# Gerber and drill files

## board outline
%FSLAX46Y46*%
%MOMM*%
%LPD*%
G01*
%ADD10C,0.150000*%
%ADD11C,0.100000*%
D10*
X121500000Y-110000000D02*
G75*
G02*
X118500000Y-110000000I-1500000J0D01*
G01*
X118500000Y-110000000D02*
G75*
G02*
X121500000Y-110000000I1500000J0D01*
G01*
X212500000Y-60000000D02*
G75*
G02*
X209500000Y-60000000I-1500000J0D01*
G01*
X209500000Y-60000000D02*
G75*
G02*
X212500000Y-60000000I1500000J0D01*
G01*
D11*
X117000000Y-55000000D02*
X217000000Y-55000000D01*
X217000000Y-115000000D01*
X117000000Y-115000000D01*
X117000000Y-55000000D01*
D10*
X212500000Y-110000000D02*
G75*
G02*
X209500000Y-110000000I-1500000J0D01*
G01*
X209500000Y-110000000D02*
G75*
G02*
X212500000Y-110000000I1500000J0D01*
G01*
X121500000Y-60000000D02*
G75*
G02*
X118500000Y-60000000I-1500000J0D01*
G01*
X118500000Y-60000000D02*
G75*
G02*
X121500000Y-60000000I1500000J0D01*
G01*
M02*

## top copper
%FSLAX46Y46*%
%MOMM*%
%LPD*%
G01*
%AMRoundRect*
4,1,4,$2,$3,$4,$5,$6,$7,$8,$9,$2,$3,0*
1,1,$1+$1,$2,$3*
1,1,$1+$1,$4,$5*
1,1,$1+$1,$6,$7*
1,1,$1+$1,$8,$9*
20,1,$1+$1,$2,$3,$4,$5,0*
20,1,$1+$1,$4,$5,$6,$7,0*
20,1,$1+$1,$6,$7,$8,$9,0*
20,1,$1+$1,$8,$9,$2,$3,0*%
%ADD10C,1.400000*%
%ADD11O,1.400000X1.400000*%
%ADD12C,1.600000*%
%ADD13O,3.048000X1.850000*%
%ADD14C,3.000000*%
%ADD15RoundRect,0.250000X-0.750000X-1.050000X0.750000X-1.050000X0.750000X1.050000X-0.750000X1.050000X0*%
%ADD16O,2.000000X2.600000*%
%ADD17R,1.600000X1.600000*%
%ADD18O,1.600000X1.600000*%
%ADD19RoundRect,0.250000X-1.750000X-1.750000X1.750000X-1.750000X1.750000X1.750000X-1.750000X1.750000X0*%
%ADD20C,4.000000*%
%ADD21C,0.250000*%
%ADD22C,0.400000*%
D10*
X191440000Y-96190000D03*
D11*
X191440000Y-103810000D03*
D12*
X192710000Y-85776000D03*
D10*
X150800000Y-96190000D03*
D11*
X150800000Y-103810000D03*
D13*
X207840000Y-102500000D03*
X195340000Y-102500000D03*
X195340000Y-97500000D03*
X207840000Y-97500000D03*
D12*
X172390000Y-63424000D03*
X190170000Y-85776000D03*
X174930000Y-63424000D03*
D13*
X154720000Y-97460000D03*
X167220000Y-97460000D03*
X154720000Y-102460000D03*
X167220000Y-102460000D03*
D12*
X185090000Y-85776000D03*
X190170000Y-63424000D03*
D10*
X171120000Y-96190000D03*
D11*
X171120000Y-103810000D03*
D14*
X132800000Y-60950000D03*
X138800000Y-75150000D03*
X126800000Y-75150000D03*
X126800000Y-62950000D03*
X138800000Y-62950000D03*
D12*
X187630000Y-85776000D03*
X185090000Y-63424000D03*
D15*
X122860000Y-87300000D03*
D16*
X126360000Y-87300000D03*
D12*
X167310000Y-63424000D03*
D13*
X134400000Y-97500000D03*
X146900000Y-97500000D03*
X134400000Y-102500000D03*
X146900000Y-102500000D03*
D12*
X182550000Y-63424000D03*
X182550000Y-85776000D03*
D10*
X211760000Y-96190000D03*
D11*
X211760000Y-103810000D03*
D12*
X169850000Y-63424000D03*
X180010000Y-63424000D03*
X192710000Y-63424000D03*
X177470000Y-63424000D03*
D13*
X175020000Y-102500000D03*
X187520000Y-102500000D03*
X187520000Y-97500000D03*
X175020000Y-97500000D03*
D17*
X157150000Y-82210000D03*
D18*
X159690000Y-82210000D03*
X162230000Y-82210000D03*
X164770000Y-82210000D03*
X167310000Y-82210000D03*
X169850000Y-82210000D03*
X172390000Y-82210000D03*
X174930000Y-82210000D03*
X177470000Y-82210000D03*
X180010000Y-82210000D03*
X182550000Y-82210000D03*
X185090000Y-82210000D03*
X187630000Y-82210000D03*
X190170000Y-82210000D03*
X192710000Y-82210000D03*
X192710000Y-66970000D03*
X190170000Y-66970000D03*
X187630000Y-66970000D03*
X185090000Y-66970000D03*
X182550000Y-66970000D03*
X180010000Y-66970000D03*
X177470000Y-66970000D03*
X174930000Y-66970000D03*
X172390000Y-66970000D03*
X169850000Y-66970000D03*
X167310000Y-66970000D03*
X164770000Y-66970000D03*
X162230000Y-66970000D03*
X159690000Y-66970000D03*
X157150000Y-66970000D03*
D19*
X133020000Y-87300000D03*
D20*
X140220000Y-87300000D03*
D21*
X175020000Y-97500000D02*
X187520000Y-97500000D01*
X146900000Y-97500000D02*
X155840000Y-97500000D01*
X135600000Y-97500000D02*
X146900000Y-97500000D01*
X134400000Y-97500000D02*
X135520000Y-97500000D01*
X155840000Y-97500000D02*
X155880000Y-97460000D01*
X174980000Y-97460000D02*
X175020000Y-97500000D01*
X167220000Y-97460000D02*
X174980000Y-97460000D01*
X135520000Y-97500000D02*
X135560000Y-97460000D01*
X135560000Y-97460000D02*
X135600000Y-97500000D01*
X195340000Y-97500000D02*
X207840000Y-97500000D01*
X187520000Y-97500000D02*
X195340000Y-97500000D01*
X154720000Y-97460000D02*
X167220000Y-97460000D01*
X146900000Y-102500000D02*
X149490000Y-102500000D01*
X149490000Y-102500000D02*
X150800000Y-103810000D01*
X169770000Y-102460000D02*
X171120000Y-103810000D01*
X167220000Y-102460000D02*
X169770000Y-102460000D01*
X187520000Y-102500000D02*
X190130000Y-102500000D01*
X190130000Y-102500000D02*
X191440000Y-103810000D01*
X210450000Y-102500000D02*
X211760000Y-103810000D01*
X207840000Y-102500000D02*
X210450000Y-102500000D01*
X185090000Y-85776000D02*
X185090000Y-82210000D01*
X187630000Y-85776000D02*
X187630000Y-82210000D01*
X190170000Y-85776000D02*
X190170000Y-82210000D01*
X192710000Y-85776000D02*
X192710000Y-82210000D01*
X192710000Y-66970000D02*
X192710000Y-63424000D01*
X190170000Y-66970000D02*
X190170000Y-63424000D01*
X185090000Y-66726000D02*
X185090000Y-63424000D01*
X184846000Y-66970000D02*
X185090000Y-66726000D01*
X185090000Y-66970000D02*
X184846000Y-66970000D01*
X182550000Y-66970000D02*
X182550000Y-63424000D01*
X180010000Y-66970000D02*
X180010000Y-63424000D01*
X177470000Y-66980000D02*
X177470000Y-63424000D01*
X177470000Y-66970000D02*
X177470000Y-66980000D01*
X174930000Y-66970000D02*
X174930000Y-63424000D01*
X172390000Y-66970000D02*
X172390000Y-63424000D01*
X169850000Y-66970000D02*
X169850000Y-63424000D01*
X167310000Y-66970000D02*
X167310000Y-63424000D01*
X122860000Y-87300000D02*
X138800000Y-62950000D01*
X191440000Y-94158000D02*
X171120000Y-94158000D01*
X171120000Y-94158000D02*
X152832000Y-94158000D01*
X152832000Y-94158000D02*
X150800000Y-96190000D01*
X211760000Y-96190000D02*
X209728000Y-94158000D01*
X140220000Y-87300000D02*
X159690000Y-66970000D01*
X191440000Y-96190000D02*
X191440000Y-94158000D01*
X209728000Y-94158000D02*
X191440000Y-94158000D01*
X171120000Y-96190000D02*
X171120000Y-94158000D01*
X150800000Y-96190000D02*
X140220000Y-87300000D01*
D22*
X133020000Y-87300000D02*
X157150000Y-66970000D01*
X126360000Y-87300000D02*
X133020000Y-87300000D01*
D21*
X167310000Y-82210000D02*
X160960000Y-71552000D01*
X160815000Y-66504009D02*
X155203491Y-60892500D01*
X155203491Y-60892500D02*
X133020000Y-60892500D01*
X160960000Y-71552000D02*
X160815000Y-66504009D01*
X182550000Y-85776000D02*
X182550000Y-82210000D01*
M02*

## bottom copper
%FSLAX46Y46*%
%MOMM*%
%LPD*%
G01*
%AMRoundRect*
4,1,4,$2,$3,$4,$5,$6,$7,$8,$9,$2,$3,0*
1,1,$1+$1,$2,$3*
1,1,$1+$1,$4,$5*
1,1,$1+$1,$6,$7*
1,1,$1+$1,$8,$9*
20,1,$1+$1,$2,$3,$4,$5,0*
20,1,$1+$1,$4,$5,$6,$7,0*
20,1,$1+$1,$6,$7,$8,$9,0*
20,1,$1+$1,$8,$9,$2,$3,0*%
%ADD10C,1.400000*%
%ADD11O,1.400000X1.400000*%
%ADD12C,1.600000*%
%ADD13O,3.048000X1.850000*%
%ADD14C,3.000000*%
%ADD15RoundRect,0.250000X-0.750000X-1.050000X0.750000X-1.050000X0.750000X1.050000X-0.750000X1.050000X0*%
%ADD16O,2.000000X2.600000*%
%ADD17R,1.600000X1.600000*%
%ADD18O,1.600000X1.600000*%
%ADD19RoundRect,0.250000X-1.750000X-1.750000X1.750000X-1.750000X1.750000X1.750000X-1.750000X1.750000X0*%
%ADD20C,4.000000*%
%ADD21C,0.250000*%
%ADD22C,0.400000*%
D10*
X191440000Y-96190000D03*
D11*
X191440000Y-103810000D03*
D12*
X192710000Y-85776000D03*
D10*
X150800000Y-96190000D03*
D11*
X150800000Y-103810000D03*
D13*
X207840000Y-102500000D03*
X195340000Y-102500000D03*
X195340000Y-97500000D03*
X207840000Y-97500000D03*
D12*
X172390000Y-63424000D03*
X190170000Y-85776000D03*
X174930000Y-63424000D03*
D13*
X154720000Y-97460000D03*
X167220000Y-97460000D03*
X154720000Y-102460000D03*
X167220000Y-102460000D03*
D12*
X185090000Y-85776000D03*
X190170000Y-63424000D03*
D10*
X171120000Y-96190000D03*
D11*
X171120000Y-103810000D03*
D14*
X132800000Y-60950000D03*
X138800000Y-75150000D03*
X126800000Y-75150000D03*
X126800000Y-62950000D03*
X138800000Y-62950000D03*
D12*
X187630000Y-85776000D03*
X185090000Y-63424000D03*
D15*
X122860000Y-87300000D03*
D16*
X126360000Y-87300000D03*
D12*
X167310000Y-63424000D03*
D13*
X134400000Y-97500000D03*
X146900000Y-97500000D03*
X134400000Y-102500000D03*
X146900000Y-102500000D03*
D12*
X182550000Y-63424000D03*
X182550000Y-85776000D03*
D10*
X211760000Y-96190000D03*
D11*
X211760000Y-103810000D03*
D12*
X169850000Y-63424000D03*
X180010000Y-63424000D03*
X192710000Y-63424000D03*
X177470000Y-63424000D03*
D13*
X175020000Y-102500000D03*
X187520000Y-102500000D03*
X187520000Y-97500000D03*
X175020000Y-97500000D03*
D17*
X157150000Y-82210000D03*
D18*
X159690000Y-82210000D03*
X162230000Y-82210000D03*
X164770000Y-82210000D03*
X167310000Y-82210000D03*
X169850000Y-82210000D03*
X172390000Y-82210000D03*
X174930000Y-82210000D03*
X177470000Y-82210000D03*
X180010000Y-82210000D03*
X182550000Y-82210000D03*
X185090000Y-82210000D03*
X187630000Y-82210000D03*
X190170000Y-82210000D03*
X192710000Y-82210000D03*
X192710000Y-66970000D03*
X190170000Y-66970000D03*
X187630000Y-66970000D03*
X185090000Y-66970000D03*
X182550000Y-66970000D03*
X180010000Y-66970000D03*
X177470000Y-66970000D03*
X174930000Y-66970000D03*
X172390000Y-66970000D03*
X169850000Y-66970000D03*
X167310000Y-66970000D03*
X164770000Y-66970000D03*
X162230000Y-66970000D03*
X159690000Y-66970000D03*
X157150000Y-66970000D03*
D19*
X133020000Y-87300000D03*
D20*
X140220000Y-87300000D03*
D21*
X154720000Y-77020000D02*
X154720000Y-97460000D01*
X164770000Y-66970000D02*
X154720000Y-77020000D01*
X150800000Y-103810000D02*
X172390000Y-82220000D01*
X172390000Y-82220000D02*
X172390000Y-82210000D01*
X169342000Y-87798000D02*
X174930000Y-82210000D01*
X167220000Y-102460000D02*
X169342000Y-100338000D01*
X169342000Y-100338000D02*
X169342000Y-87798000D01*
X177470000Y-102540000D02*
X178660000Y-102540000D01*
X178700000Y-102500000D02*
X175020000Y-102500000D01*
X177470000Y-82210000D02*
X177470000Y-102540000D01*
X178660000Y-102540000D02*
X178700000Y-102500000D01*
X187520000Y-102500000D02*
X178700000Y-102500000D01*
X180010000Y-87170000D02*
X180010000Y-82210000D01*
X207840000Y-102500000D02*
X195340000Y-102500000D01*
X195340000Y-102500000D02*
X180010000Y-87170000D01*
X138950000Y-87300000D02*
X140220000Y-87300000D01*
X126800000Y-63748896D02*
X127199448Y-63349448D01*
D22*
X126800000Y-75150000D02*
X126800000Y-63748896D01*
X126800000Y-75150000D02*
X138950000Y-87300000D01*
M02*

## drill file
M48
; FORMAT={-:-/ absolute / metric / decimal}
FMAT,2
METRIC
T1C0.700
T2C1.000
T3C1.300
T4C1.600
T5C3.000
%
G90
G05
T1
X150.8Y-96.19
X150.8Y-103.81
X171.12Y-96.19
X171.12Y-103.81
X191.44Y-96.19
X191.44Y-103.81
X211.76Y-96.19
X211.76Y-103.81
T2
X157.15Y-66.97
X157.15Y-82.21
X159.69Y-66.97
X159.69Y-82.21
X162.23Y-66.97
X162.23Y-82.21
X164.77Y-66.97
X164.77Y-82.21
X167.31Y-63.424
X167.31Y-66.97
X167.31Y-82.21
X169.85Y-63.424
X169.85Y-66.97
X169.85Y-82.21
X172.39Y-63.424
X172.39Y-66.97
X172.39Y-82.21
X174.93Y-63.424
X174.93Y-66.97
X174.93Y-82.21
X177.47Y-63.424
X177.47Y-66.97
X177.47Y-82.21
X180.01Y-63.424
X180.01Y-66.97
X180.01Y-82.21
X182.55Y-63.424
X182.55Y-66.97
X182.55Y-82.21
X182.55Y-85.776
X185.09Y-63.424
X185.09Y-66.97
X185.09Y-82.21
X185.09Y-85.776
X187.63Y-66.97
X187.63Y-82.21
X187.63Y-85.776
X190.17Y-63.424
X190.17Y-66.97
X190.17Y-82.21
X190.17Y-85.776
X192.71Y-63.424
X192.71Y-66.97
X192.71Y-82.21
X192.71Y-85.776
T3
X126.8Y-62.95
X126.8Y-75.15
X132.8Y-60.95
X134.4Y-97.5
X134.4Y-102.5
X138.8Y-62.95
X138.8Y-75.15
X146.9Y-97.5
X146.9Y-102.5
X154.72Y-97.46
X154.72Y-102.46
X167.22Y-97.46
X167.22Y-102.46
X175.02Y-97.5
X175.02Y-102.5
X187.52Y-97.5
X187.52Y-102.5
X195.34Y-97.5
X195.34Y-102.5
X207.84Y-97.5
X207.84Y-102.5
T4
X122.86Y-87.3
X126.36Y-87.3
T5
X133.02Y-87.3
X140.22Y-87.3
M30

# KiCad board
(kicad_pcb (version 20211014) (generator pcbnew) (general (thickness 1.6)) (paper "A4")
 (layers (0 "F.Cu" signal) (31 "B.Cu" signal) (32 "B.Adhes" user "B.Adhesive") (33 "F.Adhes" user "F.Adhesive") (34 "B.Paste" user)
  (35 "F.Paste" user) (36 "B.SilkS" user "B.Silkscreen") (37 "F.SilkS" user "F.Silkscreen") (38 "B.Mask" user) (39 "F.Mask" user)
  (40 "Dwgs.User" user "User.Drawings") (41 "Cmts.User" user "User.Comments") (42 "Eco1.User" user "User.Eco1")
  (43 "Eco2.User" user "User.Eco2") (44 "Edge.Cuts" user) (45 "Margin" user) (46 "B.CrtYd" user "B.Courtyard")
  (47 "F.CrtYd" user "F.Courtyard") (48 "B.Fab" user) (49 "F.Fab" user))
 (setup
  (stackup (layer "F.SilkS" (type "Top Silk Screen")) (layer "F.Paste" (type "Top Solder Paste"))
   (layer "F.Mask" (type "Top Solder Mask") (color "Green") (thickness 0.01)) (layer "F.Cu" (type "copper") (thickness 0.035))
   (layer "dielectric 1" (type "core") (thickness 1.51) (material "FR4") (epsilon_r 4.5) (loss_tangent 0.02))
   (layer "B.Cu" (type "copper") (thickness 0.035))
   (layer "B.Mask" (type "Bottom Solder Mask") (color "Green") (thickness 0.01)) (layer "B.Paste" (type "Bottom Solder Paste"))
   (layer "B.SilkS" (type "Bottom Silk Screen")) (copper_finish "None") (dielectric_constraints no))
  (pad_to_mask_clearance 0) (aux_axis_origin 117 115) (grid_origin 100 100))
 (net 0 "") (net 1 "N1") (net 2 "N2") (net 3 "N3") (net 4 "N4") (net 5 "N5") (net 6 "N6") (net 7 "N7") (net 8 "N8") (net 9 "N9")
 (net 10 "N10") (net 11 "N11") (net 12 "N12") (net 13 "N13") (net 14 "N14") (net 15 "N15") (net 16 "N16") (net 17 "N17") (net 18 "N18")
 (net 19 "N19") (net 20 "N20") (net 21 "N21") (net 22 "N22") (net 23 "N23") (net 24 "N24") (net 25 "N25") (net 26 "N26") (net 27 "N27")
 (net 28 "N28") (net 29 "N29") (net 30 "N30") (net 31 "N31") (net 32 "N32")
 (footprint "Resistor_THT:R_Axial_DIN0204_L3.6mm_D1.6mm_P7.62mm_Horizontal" (layer "F.Cu") (at 191.44 96.19 -90)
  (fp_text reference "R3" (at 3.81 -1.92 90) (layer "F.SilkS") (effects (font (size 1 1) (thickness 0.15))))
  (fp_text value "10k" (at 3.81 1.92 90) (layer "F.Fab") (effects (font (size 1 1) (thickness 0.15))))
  (pad "1" thru_hole circle (at 0 0 270) (size 1.4 1.4) (drill 0.7) (layers *.Cu *.Mask) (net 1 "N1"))
  (pad "2" thru_hole oval (at 7.62 0 270) (size 1.4 1.4) (drill 0.7) (layers *.Cu *.Mask) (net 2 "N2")))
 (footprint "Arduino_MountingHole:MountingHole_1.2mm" (layer "F.Cu") (at 192.71 85.776)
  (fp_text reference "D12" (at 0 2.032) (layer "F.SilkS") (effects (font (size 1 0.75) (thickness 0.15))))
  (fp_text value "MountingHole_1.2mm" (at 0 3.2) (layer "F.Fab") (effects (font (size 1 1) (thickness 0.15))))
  (pad "" thru_hole circle locked (at 0 0) (size 1.6 1.6) (drill 1) (layers *.Cu *.Mask) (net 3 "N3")))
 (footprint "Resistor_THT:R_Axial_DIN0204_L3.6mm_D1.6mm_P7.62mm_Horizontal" (layer "F.Cu") (at 150.8 96.19 -90)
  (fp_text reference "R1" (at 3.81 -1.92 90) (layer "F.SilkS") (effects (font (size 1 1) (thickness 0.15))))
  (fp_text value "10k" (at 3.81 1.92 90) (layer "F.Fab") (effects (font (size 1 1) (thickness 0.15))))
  (pad "1" thru_hole circle (at 0 0 270) (size 1.4 1.4) (drill 0.7) (layers *.Cu *.Mask) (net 1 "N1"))
  (pad "2" thru_hole oval (at 7.62 0 270) (size 1.4 1.4) (drill 0.7) (layers *.Cu *.Mask) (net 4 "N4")))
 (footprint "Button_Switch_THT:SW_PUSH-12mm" (layer "F.Cu") (at 207.84 102.5 180)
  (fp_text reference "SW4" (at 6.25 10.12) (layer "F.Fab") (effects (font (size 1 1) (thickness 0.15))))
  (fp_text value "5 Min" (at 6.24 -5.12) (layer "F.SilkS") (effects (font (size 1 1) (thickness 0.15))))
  (pad "1" thru_hole oval (at 0 0 180) (size 3.048 1.85) (drill 1.3) (layers *.Cu *.Mask) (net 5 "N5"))
  (pad "1" thru_hole oval (at 12.5 0 180) (size 3.048 1.85) (drill 1.3) (layers *.Cu *.Mask) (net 5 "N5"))
  (pad "2" thru_hole oval (at 12.5 5 180) (size 3.048 1.85) (drill 1.3) (layers *.Cu *.Mask) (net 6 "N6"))
  (pad "2" thru_hole oval (at 0 5 180) (size 3.048 1.85) (drill 1.3) (layers *.Cu *.Mask) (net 6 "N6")))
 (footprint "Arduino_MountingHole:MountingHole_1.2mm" (layer "F.Cu") (at 172.39 63.424)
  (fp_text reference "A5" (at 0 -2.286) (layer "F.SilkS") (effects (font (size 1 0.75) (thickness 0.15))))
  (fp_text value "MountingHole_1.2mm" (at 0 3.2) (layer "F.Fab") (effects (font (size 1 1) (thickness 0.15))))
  (pad "" thru_hole circle locked (at 0 0) (size 1.6 1.6) (drill 1) (layers *.Cu *.Mask) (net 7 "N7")))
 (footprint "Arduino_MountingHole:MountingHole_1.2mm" (layer "F.Cu") (at 190.17 85.776)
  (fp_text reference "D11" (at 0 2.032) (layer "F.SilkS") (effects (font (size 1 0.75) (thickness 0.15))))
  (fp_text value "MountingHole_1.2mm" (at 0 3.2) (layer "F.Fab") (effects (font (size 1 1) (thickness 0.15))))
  (pad "" thru_hole circle locked (at 0 0) (size 1.6 1.6) (drill 1) (layers *.Cu *.Mask) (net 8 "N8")))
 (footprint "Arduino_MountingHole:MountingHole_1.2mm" (layer "F.Cu") (at 174.93 63.424)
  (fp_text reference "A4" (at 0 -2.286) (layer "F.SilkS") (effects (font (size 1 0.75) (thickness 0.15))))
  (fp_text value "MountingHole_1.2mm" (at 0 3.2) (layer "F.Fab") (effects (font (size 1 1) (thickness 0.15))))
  (pad "" thru_hole circle locked (at 0 0) (size 1.6 1.6) (drill 1) (layers *.Cu *.Mask) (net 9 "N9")))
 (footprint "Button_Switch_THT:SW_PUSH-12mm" (layer "F.Cu") (at 154.72 97.46)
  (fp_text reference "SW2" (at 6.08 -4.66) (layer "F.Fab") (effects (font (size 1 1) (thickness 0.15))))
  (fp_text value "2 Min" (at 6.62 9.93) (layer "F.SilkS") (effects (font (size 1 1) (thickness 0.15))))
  (pad "1" thru_hole oval (at 0 0) (size 3.048 1.85) (drill 1.3) (layers *.Cu *.Mask) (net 6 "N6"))
  (pad "1" thru_hole oval (at 12.5 0) (size 3.048 1.85) (drill 1.3) (layers *.Cu *.Mask) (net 6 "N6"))
  (pad "2" thru_hole oval (at 0 5) (size 3.048 1.85) (drill 1.3) (layers *.Cu *.Mask) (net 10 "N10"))
  (pad "2" thru_hole oval (at 12.5 5) (size 3.048 1.85) (drill 1.3) (layers *.Cu *.Mask) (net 10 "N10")))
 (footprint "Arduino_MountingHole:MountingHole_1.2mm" (layer "F.Cu") (at 185.09 85.776)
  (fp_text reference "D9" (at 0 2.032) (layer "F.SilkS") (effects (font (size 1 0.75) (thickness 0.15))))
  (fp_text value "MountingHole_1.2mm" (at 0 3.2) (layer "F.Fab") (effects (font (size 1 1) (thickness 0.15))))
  (pad "" thru_hole circle locked (at 0 0) (size 1.6 1.6) (drill 1) (layers *.Cu *.Mask) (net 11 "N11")))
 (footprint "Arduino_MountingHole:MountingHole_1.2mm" (layer "F.Cu") (at 190.17 63.424)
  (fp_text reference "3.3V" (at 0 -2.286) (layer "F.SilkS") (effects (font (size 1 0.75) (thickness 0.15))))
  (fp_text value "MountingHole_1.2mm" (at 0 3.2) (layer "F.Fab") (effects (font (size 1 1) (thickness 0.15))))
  (pad "" thru_hole circle locked (at 0 0) (size 1.6 1.6) (drill 1) (layers *.Cu *.Mask) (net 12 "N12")))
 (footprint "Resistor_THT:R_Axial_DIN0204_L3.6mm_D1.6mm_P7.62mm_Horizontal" (layer "F.Cu") (at 171.12 96.19 -90)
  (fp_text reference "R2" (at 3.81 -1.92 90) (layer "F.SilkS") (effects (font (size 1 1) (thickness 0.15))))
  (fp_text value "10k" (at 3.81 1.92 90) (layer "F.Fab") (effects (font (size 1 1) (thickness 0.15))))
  (pad "1" thru_hole circle (at 0 0 270) (size 1.4 1.4) (drill 0.7) (layers *.Cu *.Mask) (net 1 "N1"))
  (pad "2" thru_hole oval (at 7.62 0 270) (size 1.4 1.4) (drill 0.7) (layers *.Cu *.Mask) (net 10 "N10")))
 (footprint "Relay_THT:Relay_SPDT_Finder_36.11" (layer "F.Cu") (at 132.8 60.95 -90)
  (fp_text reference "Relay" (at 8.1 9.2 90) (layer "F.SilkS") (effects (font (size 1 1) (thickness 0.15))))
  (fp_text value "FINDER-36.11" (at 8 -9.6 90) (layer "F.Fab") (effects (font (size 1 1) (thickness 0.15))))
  (pad "11" thru_hole circle (at 0 0 270) (size 3 3) (drill 1.3) (layers *.Cu *.Mask) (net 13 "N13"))
  (pad "12" thru_hole circle (at 14.2 -6 270) (size 3 3) (drill 1.3) (layers *.Cu *.Mask) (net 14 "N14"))
  (pad "14" thru_hole circle (at 14.2 6 270) (size 3 3) (drill 1.3) (layers *.Cu *.Mask) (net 1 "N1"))
  (pad "A1" thru_hole circle (at 2 6 270) (size 3 3) (drill 1.3) (layers *.Cu *.Mask) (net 1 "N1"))
  (pad "A2" thru_hole circle (at 2 -6 270) (size 3 3) (drill 1.3) (layers *.Cu *.Mask) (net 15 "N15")))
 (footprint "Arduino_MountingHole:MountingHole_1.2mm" (layer "F.Cu") (at 187.63 85.776)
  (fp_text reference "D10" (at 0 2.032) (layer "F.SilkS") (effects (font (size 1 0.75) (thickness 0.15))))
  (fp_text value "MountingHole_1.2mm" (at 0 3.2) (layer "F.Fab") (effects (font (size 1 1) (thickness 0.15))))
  (pad "" thru_hole circle locked (at 0 0) (size 1.6 1.6) (drill 1) (layers *.Cu *.Mask) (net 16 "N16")))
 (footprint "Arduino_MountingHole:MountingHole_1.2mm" (layer "F.Cu") (at 185.09 63.424)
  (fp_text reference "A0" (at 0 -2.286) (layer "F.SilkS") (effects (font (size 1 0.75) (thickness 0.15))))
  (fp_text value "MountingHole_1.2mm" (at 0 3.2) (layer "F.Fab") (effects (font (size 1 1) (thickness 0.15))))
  (pad "" thru_hole circle locked (at 0 0) (size 1.6 1.6) (drill 1) (layers *.Cu *.Mask) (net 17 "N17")))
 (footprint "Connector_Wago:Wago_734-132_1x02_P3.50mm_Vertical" (layer "F.Cu") (at 122.86 87.3)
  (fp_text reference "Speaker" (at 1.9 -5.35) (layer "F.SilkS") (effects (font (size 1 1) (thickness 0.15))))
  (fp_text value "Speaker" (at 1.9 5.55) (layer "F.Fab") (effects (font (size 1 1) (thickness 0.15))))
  (pad "1" thru_hole roundrect (at 0 0) (size 2 2.6) (drill 1.6) (layers *.Cu *.Mask) (roundrect_rratio 0.125) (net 15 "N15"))
  (pad "2" thru_hole oval (at 3.5 0) (size 2 2.6) (drill 1.6) (layers *.Cu *.Mask) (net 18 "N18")))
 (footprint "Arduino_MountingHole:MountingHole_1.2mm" (layer "F.Cu") (at 167.31 63.424)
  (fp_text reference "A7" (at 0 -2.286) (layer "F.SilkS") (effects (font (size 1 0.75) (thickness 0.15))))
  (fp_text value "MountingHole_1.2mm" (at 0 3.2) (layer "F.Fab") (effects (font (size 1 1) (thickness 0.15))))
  (pad "" thru_hole circle locked (at 0 0) (size 1.6 1.6) (drill 1) (layers *.Cu *.Mask) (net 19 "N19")))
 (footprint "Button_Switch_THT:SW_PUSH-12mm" (layer "F.Cu") (at 134.4 97.5)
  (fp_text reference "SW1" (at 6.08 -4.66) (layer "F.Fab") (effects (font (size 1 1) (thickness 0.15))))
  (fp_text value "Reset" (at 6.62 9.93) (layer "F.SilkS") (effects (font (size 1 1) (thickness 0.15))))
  (pad "1" thru_hole oval (at 0 0) (size 3.048 1.85) (drill 1.3) (layers *.Cu *.Mask) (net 6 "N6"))
  (pad "1" thru_hole oval (at 12.5 0) (size 3.048 1.85) (drill 1.3) (layers *.Cu *.Mask) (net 6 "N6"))
  (pad "2" thru_hole oval (at 0 5) (size 3.048 1.85) (drill 1.3) (layers *.Cu *.Mask) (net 4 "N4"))
  (pad "2" thru_hole oval (at 12.5 5) (size 3.048 1.85) (drill 1.3) (layers *.Cu *.Mask) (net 4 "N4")))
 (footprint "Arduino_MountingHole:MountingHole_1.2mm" (layer "F.Cu") (at 182.55 63.424)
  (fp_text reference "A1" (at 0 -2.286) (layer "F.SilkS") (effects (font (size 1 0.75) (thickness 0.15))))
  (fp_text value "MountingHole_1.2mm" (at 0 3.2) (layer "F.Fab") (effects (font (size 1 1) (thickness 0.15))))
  (pad "" thru_hole circle locked (at 0 0) (size 1.6 1.6) (drill 1) (layers *.Cu *.Mask) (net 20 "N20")))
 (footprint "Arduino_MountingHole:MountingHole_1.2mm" (layer "F.Cu") (at 182.55 85.776)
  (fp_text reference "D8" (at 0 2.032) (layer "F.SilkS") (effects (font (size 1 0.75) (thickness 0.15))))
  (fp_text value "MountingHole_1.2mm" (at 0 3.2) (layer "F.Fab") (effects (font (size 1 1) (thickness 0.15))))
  (pad "" thru_hole circle locked (at 0 0) (size 1.6 1.6) (drill 1) (layers *.Cu *.Mask) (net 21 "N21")))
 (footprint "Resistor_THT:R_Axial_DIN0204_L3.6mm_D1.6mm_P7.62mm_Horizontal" (layer "F.Cu") (at 211.76 96.19 -90)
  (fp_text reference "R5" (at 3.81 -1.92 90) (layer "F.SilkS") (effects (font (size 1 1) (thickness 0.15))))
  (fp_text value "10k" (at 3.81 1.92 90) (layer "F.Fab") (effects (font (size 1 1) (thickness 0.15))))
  (pad "1" thru_hole circle (at 0 0 270) (size 1.4 1.4) (drill 0.7) (layers *.Cu *.Mask) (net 1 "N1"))
  (pad "2" thru_hole oval (at 7.62 0 270) (size 1.4 1.4) (drill 0.7) (layers *.Cu *.Mask) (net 5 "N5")))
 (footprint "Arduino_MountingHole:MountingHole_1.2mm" (layer "F.Cu") (at 169.85 63.424)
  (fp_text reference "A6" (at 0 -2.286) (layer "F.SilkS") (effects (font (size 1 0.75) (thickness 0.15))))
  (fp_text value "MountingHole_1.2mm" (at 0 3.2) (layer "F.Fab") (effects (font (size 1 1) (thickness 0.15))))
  (pad "" thru_hole circle locked (at 0 0) (size 1.6 1.6) (drill 1) (layers *.Cu *.Mask) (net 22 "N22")))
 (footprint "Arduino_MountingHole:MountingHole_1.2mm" (layer "F.Cu") (at 180.01 63.424)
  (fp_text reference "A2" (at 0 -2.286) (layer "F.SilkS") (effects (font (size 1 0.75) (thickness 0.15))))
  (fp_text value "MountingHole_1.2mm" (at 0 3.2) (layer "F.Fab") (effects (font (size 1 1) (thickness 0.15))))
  (pad "" thru_hole circle locked (at 0 0) (size 1.6 1.6) (drill 1) (layers *.Cu *.Mask) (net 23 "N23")))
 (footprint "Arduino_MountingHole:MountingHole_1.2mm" (layer "F.Cu") (at 192.71 63.424)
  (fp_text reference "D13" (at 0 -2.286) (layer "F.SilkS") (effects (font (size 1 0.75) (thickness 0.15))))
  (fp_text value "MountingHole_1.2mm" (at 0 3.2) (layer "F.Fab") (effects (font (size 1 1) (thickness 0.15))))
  (pad "" thru_hole circle locked (at 0 0) (size 1.6 1.6) (drill 1) (layers *.Cu *.Mask) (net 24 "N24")))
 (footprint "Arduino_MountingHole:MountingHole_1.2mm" (layer "F.Cu") (at 177.47 63.424)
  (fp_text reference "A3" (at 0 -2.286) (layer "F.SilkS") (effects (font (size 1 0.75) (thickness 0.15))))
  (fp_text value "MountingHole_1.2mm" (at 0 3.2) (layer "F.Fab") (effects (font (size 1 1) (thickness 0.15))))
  (pad "" thru_hole circle locked (at 0 0) (size 1.6 1.6) (drill 1) (layers *.Cu *.Mask) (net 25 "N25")))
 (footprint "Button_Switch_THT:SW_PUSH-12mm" (layer "F.Cu") (at 187.52 102.5 180)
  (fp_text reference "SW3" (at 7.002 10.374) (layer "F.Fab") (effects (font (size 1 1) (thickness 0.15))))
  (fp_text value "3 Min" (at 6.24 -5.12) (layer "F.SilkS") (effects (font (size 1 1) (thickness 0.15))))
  (pad "1" thru_hole oval (at 12.5 0 180) (size 3.048 1.85) (drill 1.3) (layers *.Cu *.Mask) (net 2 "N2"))
  (pad "1" thru_hole oval (at 0 0 180) (size 3.048 1.85) (drill 1.3) (layers *.Cu *.Mask) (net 2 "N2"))
  (pad "2" thru_hole oval (at 0 5 180) (size 3.048 1.85) (drill 1.3) (layers *.Cu *.Mask) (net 6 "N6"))
  (pad "2" thru_hole oval (at 12.5 5 180) (size 3.048 1.85) (drill 1.3) (layers *.Cu *.Mask) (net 6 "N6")))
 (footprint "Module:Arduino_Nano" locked (layer "F.Cu") (at 157.15 82.21 90)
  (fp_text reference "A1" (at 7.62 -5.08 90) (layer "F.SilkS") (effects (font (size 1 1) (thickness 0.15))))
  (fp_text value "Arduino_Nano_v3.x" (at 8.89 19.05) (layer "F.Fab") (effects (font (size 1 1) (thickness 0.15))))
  (pad "1" thru_hole rect locked (at 0 0 90) (size 1.6 1.6) (drill 1) (layers *.Cu *.Mask) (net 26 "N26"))
  (pad "2" thru_hole oval locked (at 0 2.54 90) (size 1.6 1.6) (drill 1) (layers *.Cu *.Mask) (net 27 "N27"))
  (pad "3" thru_hole oval locked (at 0 5.08 90) (size 1.6 1.6) (drill 1) (layers *.Cu *.Mask) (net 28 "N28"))
  (pad "4" thru_hole oval locked (at 0 7.62 90) (size 1.6 1.6) (drill 1) (layers *.Cu *.Mask) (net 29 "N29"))
  (pad "5" thru_hole oval locked (at 0 10.16 90) (size 1.6 1.6) (drill 1) (layers *.Cu *.Mask) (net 13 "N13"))
  (pad "6" thru_hole oval locked (at 0 12.7 90) (size 1.6 1.6) (drill 1) (layers *.Cu *.Mask) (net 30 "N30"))
  (pad "7" thru_hole oval locked (at 0 15.24 90) (size 1.6 1.6) (drill 1) (layers *.Cu *.Mask) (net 4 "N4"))
  (pad "8" thru_hole oval locked (at 0 17.78 90) (size 1.6 1.6) (drill 1) (layers *.Cu *.Mask) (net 10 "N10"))
  (pad "9" thru_hole oval locked (at 0 20.32 90) (size 1.6 1.6) (drill 1) (layers *.Cu *.Mask) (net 2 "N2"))
  (pad "10" thru_hole oval locked (at 0 22.86 90) (size 1.6 1.6) (drill 1) (layers *.Cu *.Mask) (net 5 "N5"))
  (pad "11" thru_hole oval locked (at 0 25.4 90) (size 1.6 1.6) (drill 1) (layers *.Cu *.Mask) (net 21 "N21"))
  (pad "12" thru_hole oval locked (at 0 27.94 90) (size 1.6 1.6) (drill 1) (layers *.Cu *.Mask) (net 11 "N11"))
  (pad "13" thru_hole oval locked (at 0 30.48 90) (size 1.6 1.6) (drill 1) (layers *.Cu *.Mask) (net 16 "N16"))
  (pad "14" thru_hole oval locked (at 0 33.02 90) (size 1.6 1.6) (drill 1) (layers *.Cu *.Mask) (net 8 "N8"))
  (pad "15" thru_hole oval locked (at 0 35.56 90) (size 1.6 1.6) (drill 1) (layers *.Cu *.Mask) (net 3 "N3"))
  (pad "16" thru_hole oval locked (at 15.24 35.56 90) (size 1.6 1.6) (drill 1) (layers *.Cu *.Mask) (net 24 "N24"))
  (pad "17" thru_hole oval locked (at 15.24 33.02 90) (size 1.6 1.6) (drill 1) (layers *.Cu *.Mask) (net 12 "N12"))
  (pad "18" thru_hole oval locked (at 15.24 30.48 90) (size 1.6 1.6) (drill 1) (layers *.Cu *.Mask) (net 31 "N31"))
  (pad "19" thru_hole oval locked (at 15.24 27.94 90) (size 1.6 1.6) (drill 1) (layers *.Cu *.Mask) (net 17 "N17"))
  (pad "20" thru_hole oval locked (at 15.24 25.4 90) (size 1.6 1.6) (drill 1) (layers *.Cu *.Mask) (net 20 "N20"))
  (pad "21" thru_hole oval locked (at 15.24 22.86 90) (size 1.6 1.6) (drill 1) (layers *.Cu *.Mask) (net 23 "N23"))
  (pad "22" thru_hole oval locked (at 15.24 20.32 90) (size 1.6 1.6) (drill 1) (layers *.Cu *.Mask) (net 25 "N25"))
  (pad "23" thru_hole oval locked (at 15.24 17.78 90) (size 1.6 1.6) (drill 1) (layers *.Cu *.Mask) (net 9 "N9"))
  (pad "24" thru_hole oval locked (at 15.24 15.24 90) (size 1.6 1.6) (drill 1) (layers *.Cu *.Mask) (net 7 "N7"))
  (pad "25" thru_hole oval locked (at 15.24 12.7 90) (size 1.6 1.6) (drill 1) (layers *.Cu *.Mask) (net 22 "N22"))
  (pad "26" thru_hole oval locked (at 15.24 10.16 90) (size 1.6 1.6) (drill 1) (layers *.Cu *.Mask) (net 19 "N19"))
  (pad "27" thru_hole oval locked (at 15.24 7.62 90) (size 1.6 1.6) (drill 1) (layers *.Cu *.Mask) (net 6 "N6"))
  (pad "28" thru_hole oval locked (at 15.24 5.08 90) (size 1.6 1.6) (drill 1) (layers *.Cu *.Mask) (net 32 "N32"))
  (pad "29" thru_hole oval locked (at 15.24 2.54 90) (size 1.6 1.6) (drill 1) (layers *.Cu *.Mask) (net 1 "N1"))
  (pad "30" thru_hole oval locked (at 15.24 0 90) (size 1.6 1.6) (drill 1) (layers *.Cu *.Mask) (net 18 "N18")))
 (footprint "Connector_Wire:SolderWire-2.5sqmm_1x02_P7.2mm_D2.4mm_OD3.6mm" (layer "F.Cu") (at 133.02 87.3)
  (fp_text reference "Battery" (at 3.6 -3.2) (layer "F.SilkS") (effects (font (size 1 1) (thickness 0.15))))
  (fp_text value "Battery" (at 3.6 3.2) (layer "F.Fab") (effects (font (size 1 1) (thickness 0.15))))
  (pad "1" thru_hole roundrect (at 0 0) (size 4 4) (drill 3) (layers *.Cu *.Mask) (roundrect_rratio 0.0625) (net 18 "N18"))
  (pad "2" thru_hole circle (at 7.2 0) (size 4 4) (drill 3) (layers *.Cu *.Mask) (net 1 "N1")))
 (gr_circle (center 120 110) (end 121.5 110) (layer "Edge.Cuts") (width 0.15) (fill none))
 (gr_circle (center 211 60) (end 212.5 60) (layer "Edge.Cuts") (width 0.15) (fill none))
 (gr_rect (start 117 55) (end 217 115) (layer "Edge.Cuts") (width 0.1) (fill none))
 (gr_circle (center 211 110) (end 212.5 110) (layer "Edge.Cuts") (width 0.15) (fill none))
 (gr_circle (center 120 60) (end 121.5 60) (layer "Edge.Cuts") (width 0.15) (fill none))
 (segment (start 175.02 97.5) (end 187.52 97.5) (width 0.25) (layer "F.Cu") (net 6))
 (segment (start 146.9 97.5) (end 155.84 97.5) (width 0.25) (layer "F.Cu") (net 6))
 (segment (start 135.6 97.5) (end 146.9 97.5) (width 0.25) (layer "F.Cu") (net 6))
 (segment (start 134.4 97.5) (end 135.52 97.5) (width 0.25) (layer "F.Cu") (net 6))
 (segment (start 155.84 97.5) (end 155.88 97.46) (width 0.25) (layer "F.Cu") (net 6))
 (segment (start 174.98 97.46) (end 175.02 97.5) (width 0.25) (layer "F.Cu") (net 6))
 (segment (start 167.22 97.46) (end 174.98 97.46) (width 0.25) (layer "F.Cu") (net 6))
 (segment (start 135.52 97.5) (end 135.56 97.46) (width 0.25) (layer "F.Cu") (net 6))
 (segment (start 135.56 97.46) (end 135.6 97.5) (width 0.25) (layer "F.Cu") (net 6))
 (segment (start 195.34 97.5) (end 207.84 97.5) (width 0.25) (layer "F.Cu") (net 6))
 (segment (start 187.52 97.5) (end 195.34 97.5) (width 0.25) (layer "F.Cu") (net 6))
 (segment (start 154.72 97.46) (end 167.22 97.46) (width 0.25) (layer "F.Cu") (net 6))
 (segment (start 154.72 77.02) (end 154.72 97.46) (width 0.25) (layer "B.Cu") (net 6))
 (segment (start 164.77 66.97) (end 154.72 77.02) (width 0.25) (layer "B.Cu") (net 6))
 (segment (start 146.9 102.5) (end 149.49 102.5) (width 0.25) (layer "F.Cu") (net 4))
 (segment (start 149.49 102.5) (end 150.8 103.81) (width 0.25) (layer "F.Cu") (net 4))
 (segment (start 150.8 103.81) (end 172.39 82.22) (width 0.25) (layer "B.Cu") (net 4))
 (segment (start 172.39 82.22) (end 172.39 82.21) (width 0.25) (layer "B.Cu") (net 4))
 (segment (start 169.77 102.46) (end 171.12 103.81) (width 0.25) (layer "F.Cu") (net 10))
 (segment (start 167.22 102.46) (end 169.77 102.46) (width 0.25) (layer "F.Cu") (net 10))
 (segment (start 169.342 87.798) (end 174.93 82.21) (width 0.25) (layer "B.Cu") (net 10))
 (segment (start 167.22 102.46) (end 169.342 100.338) (width 0.25) (layer "B.Cu") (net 10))
 (segment (start 169.342 100.338) (end 169.342 87.798) (width 0.25) (layer "B.Cu") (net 10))
 (segment (start 187.52 102.5) (end 190.13 102.5) (width 0.25) (layer "F.Cu") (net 2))
 (segment (start 190.13 102.5) (end 191.44 103.81) (width 0.25) (layer "F.Cu") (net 2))
 (segment (start 177.47 102.54) (end 178.66 102.54) (width 0.25) (layer "B.Cu") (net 2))
 (segment (start 178.7 102.5) (end 175.02 102.5) (width 0.25) (layer "B.Cu") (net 2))
 (segment (start 177.47 82.21) (end 177.47 102.54) (width 0.25) (layer "B.Cu") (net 2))
 (segment (start 178.66 102.54) (end 178.7 102.5) (width 0.25) (layer "B.Cu") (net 2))
 (segment (start 187.52 102.5) (end 178.7 102.5) (width 0.25) (layer "B.Cu") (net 2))
 (segment (start 210.45 102.5) (end 211.76 103.81) (width 0.25) (layer "F.Cu") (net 5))
 (segment (start 207.84 102.5) (end 210.45 102.5) (width 0.25) (layer "F.Cu") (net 5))
 (segment (start 180.01 87.17) (end 180.01 82.21) (width 0.25) (layer "B.Cu") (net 5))
 (segment (start 207.84 102.5) (end 195.34 102.5) (width 0.25) (layer "B.Cu") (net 5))
 (segment (start 195.34 102.5) (end 180.01 87.17) (width 0.25) (layer "B.Cu") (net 5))
 (segment (start 185.09 85.776) (end 185.09 82.21) (width 0.25) (layer "F.Cu") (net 11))
 (segment (start 187.63 85.776) (end 187.63 82.21) (width 0.25) (layer "F.Cu") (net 16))
 (segment (start 190.17 85.776) (end 190.17 82.21) (width 0.25) (layer "F.Cu") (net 8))
 (segment (start 192.71 85.776) (end 192.71 82.21) (width 0.25) (layer "F.Cu") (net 3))
 (segment (start 192.71 66.97) (end 192.71 63.424) (width 0.25) (layer "F.Cu") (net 24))
 (segment (start 190.17 66.97) (end 190.17 63.424) (width 0.25) (layer "F.Cu") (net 12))
 (segment (start 185.09 66.726) (end 185.09 63.424) (width 0.25) (layer "F.Cu") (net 17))
 (segment (start 184.846 66.97) (end 185.09 66.726) (width 0.25) (layer "F.Cu") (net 17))
 (segment (start 185.09 66.97) (end 184.846 66.97) (width 0.25) (layer "F.Cu") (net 17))
 (segment (start 182.55 66.97) (end 182.55 63.424) (width 0.25) (layer "F.Cu") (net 20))
 (segment (start 180.01 66.97) (end 180.01 63.424) (width 0.25) (layer "F.Cu") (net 23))
 (segment (start 177.47 66.98) (end 177.47 63.424) (width 0.25) (layer "F.Cu") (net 25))
 (segment (start 177.47 66.97) (end 177.47 66.98) (width 0.25) (layer "F.Cu") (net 25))
 (segment (start 174.93 66.97) (end 174.93 63.424) (width 0.25) (layer "F.Cu") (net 9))
 (segment (start 172.39 66.97) (end 172.39 63.424) (width 0.25) (layer "F.Cu") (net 7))
 (segment (start 169.85 66.97) (end 169.85 63.424) (width 0.25) (layer "F.Cu") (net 22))
 (segment (start 167.31 66.97) (end 167.31 63.424) (width 0.25) (layer "F.Cu") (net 19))
 (segment (start 122.86 87.3) (end 138.8 62.95) (width 0.25) (layer "F.Cu") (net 15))
 (segment (start 191.44 94.158) (end 171.12 94.158) (width 0.25) (layer "F.Cu") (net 1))
 (segment (start 171.12 94.158) (end 152.832 94.158) (width 0.25) (layer "F.Cu") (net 1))
 (segment (start 152.832 94.158) (end 150.8 96.19) (width 0.25) (layer "F.Cu") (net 1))
 (segment (start 211.76 96.19) (end 209.728 94.158) (width 0.25) (layer "F.Cu") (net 1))
 (segment (start 140.22 87.3) (end 159.69 66.97) (width 0.25) (layer "F.Cu") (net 1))
 (segment (start 191.44 96.19) (end 191.44 94.158) (width 0.25) (layer "F.Cu") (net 1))
 (segment (start 209.728 94.158) (end 191.44 94.158) (width 0.25) (layer "F.Cu") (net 1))
 (segment (start 171.12 96.19) (end 171.12 94.158) (width 0.25) (layer "F.Cu") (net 1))
 (segment (start 150.8 96.19) (end 140.22 87.3) (width 0.25) (layer "F.Cu") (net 1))
 (segment (start 138.95 87.3) (end 140.22 87.3) (width 0.25) (layer "B.Cu") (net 1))
 (segment (start 126.8 63.748896) (end 127.199448 63.349448) (width 0.25) (layer "B.Cu") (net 1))
 (segment (start 126.8 75.15) (end 126.8 63.748896) (width 0.4) (layer "B.Cu") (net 1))
 (segment (start 126.8 75.15) (end 138.95 87.3) (width 0.4) (layer "B.Cu") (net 1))
 (segment (start 133.02 87.3) (end 157.15 66.97) (width 0.4) (layer "F.Cu") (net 18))
 (segment (start 126.36 87.3) (end 133.02 87.3) (width 0.4) (layer "F.Cu") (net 18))
 (segment (start 167.31 82.21) (end 160.96 71.552) (width 0.25) (layer "F.Cu") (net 13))
 (segment (start 160.815 66.504009) (end 155.203491 60.8925) (width 0.25) (layer "F.Cu") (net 13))
 (segment (start 155.203491 60.8925) (end 133.02 60.8925) (width 0.25) (layer "F.Cu") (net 13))
 (segment (start 160.96 71.552) (end 160.815 66.504009) (width 0.25) (layer "F.Cu") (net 13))
 (segment (start 182.55 85.776) (end 182.55 82.21) (width 0.25) (layer "F.Cu") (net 21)))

